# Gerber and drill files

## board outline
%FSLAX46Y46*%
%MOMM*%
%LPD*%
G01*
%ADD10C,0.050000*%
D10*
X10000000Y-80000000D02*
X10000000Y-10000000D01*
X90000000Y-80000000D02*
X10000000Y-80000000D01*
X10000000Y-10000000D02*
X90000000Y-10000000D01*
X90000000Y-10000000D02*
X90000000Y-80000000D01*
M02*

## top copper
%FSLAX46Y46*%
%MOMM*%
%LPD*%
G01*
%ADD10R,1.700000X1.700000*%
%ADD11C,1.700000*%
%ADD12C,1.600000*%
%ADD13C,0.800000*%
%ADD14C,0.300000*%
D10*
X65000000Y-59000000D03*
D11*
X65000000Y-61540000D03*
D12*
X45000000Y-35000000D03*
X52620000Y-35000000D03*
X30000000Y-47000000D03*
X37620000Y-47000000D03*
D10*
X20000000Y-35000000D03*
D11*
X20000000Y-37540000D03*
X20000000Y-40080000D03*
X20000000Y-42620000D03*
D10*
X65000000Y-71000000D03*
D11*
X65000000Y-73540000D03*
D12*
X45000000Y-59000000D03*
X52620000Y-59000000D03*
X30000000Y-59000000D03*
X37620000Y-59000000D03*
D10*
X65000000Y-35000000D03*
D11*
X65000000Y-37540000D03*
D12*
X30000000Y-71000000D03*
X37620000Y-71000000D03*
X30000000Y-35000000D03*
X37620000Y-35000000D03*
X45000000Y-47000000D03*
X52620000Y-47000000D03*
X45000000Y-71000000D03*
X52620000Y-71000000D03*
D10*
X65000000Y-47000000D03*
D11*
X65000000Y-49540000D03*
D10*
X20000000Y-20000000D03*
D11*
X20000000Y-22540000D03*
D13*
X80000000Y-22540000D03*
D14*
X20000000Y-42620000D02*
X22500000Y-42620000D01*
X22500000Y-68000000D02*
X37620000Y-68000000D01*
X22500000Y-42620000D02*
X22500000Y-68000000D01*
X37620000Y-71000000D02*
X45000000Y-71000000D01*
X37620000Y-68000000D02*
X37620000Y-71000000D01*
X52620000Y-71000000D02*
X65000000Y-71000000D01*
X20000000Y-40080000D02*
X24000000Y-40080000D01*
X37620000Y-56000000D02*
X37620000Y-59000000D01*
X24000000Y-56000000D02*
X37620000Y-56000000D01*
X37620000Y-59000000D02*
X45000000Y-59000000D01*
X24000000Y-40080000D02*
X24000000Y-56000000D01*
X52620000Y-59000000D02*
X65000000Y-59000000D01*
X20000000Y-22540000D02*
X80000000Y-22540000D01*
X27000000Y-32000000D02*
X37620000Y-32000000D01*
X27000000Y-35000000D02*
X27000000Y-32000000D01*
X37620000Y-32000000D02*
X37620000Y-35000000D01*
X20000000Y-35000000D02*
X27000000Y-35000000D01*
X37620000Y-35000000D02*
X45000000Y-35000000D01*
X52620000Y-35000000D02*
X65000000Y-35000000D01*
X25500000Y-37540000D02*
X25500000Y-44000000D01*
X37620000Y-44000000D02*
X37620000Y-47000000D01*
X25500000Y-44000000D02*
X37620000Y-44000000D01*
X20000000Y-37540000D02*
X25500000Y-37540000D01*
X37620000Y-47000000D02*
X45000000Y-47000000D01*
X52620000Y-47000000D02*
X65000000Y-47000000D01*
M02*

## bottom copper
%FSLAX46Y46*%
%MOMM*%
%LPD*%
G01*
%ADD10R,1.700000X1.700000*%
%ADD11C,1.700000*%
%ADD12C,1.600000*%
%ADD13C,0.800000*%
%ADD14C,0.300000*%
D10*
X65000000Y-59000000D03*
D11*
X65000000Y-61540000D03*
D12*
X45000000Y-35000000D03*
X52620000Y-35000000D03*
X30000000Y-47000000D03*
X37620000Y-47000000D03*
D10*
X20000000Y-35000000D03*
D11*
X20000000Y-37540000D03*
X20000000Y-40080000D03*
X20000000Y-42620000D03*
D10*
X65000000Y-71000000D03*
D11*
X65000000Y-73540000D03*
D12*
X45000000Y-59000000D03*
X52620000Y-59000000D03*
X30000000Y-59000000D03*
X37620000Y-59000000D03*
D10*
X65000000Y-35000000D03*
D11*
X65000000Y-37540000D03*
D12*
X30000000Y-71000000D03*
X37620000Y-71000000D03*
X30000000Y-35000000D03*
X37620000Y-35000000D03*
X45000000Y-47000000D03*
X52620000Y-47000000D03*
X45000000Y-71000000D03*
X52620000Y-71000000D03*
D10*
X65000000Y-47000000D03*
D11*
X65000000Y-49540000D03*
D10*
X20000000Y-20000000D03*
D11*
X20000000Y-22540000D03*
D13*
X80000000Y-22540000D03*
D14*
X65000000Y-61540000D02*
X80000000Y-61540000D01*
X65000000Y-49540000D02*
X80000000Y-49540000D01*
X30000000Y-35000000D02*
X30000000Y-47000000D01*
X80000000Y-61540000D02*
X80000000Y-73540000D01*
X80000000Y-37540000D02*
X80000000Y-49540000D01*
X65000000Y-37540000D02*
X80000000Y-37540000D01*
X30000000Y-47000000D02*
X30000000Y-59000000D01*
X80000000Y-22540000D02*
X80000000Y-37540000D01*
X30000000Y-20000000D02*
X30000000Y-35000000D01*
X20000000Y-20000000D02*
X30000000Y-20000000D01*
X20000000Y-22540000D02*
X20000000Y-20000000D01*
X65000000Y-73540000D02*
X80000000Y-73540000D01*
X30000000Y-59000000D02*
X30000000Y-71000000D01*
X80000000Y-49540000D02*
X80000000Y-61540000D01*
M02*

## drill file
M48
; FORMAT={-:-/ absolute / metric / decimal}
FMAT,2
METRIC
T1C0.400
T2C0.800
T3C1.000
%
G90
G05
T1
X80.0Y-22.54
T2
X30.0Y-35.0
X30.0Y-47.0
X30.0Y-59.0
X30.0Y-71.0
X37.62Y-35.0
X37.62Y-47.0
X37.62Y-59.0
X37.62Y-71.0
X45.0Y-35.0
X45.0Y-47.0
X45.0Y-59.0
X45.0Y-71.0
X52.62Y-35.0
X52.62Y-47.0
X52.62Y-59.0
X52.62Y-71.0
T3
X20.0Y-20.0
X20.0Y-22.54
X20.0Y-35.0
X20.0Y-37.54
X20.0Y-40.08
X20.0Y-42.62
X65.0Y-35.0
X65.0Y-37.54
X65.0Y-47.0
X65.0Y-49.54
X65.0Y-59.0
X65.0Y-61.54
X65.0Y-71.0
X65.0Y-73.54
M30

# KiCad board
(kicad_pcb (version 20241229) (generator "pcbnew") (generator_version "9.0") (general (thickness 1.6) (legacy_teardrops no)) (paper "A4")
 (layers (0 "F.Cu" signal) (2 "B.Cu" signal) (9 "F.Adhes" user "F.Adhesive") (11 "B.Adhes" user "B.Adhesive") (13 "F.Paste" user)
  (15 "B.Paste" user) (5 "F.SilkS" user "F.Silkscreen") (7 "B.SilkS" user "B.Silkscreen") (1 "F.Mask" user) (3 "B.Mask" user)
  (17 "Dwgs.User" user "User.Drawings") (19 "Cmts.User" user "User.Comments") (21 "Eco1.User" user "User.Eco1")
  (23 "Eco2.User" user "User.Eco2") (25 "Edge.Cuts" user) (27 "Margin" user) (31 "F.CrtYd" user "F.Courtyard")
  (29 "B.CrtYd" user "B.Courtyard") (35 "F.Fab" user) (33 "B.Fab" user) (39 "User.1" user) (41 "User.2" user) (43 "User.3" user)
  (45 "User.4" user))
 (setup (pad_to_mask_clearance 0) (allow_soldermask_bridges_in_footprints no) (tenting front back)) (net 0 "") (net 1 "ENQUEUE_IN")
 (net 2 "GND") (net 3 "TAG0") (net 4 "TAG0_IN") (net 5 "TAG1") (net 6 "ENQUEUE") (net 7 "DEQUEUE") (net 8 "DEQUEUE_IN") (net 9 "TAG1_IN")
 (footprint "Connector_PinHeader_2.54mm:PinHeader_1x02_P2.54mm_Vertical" (layer "F.Cu") (at 65 59)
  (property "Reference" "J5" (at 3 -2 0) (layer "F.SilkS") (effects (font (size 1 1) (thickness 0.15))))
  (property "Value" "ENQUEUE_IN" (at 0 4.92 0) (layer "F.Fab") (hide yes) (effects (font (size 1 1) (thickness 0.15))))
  (pad "1" thru_hole rect (at 0 0) (size 1.7 1.7) (drill 1) (layers "*.Cu" "*.Mask") (remove_unused_layers no) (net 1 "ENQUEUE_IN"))
  (pad "2" thru_hole circle (at 0 2.54) (size 1.7 1.7) (drill 1) (layers "*.Cu" "*.Mask") (remove_unused_layers no) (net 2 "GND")))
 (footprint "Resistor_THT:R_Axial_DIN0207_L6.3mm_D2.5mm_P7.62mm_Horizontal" (layer "F.Cu") (at 45 35)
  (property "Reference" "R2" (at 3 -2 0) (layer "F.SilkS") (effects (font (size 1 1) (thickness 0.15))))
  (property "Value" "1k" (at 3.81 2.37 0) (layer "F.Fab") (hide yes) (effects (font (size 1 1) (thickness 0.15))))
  (pad "1" thru_hole circle (at 0 0) (size 1.6 1.6) (drill 0.8) (layers "*.Cu" "*.Mask") (remove_unused_layers no) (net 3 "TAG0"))
  (pad "2" thru_hole circle (at 7.62 0) (size 1.6 1.6) (drill 0.8) (layers "*.Cu" "*.Mask") (remove_unused_layers no) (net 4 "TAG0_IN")))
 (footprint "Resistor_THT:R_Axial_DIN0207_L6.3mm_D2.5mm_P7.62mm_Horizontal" (layer "F.Cu") (at 30 47)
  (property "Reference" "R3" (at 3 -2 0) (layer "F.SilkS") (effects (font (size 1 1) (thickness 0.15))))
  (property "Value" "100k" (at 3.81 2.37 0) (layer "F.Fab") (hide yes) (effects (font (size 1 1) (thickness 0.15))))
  (pad "1" thru_hole circle (at 0 0) (size 1.6 1.6) (drill 0.8) (layers "*.Cu" "*.Mask") (remove_unused_layers no) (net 2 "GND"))
  (pad "2" thru_hole circle (at 7.62 0) (size 1.6 1.6) (drill 0.8) (layers "*.Cu" "*.Mask") (remove_unused_layers no) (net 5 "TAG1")))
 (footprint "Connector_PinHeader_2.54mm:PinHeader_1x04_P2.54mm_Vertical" (layer "F.Cu") (at 20 35)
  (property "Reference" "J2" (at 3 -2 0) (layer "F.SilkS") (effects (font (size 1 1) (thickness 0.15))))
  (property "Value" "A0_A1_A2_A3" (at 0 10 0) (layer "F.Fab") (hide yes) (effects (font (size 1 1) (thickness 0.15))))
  (pad "1" thru_hole rect (at 0 0) (size 1.7 1.7) (drill 1) (layers "*.Cu" "*.Mask") (remove_unused_layers no) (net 3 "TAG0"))
  (pad "2" thru_hole circle (at 0 2.54) (size 1.7 1.7) (drill 1) (layers "*.Cu" "*.Mask") (remove_unused_layers no) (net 5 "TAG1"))
  (pad "3" thru_hole circle (at 0 5.08) (size 1.7 1.7) (drill 1) (layers "*.Cu" "*.Mask") (remove_unused_layers no) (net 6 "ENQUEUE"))
  (pad "4" thru_hole circle (at 0 7.62) (size 1.7 1.7) (drill 1) (layers "*.Cu" "*.Mask") (remove_unused_layers no) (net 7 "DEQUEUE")))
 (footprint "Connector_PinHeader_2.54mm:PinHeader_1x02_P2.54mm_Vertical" (layer "F.Cu") (at 65 71)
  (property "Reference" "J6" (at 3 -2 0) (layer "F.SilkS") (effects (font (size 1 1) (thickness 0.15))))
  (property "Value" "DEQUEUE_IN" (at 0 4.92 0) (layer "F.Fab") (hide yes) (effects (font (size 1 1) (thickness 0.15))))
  (pad "1" thru_hole rect (at 0 0) (size 1.7 1.7) (drill 1) (layers "*.Cu" "*.Mask") (remove_unused_layers no) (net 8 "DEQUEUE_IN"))
  (pad "2" thru_hole circle (at 0 2.54) (size 1.7 1.7) (drill 1) (layers "*.Cu" "*.Mask") (remove_unused_layers no) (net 2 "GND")))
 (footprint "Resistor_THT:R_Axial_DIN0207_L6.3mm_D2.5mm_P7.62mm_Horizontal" (layer "F.Cu") (at 45 59)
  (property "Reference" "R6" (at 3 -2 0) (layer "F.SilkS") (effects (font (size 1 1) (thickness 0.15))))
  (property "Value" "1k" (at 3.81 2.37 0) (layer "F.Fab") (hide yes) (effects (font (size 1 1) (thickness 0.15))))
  (pad "1" thru_hole circle (at 0 0) (size 1.6 1.6) (drill 0.8) (layers "*.Cu" "*.Mask") (remove_unused_layers no) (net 6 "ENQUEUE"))
  (pad "2" thru_hole circle (at 7.62 0) (size 1.6 1.6) (drill 0.8) (layers "*.Cu" "*.Mask") (remove_unused_layers no) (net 1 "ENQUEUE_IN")))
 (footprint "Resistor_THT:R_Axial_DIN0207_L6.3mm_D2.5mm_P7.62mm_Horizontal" (layer "F.Cu") (at 30 59)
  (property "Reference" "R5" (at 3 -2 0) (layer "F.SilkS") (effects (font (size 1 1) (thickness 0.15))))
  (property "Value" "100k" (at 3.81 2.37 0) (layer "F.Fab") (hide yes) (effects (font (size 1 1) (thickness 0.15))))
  (pad "1" thru_hole circle (at 0 0) (size 1.6 1.6) (drill 0.8) (layers "*.Cu" "*.Mask") (remove_unused_layers no) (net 2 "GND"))
  (pad "2" thru_hole circle (at 7.62 0) (size 1.6 1.6) (drill 0.8) (layers "*.Cu" "*.Mask") (remove_unused_layers no) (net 6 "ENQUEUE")))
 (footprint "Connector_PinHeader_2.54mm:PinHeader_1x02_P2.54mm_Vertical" (layer "F.Cu") (at 65 35)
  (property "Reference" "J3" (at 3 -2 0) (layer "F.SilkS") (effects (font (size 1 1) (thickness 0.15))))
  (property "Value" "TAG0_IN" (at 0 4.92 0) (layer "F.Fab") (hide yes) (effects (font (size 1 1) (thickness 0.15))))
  (pad "1" thru_hole rect (at 0 0) (size 1.7 1.7) (drill 1) (layers "*.Cu" "*.Mask") (remove_unused_layers no) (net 4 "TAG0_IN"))
  (pad "2" thru_hole circle (at 0 2.54) (size 1.7 1.7) (drill 1) (layers "*.Cu" "*.Mask") (remove_unused_layers no) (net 2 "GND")))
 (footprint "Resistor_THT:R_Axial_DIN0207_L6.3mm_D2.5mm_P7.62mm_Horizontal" (layer "F.Cu") (at 30 71)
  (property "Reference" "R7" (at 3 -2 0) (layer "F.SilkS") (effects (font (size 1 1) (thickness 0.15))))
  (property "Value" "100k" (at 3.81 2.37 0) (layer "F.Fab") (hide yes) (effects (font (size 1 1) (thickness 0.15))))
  (pad "1" thru_hole circle (at 0 0) (size 1.6 1.6) (drill 0.8) (layers "*.Cu" "*.Mask") (remove_unused_layers no) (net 2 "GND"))
  (pad "2" thru_hole circle (at 7.62 0) (size 1.6 1.6) (drill 0.8) (layers "*.Cu" "*.Mask") (remove_unused_layers no) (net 7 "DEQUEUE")))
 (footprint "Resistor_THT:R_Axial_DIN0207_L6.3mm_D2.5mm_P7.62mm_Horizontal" (layer "F.Cu") (at 30 35)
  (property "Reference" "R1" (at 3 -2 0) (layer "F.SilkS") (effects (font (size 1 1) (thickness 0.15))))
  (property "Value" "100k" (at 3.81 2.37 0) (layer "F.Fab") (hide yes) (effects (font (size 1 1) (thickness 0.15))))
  (pad "1" thru_hole circle (at 0 0) (size 1.6 1.6) (drill 0.8) (layers "*.Cu" "*.Mask") (remove_unused_layers no) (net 2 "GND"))
  (pad "2" thru_hole circle (at 7.62 0) (size 1.6 1.6) (drill 0.8) (layers "*.Cu" "*.Mask") (remove_unused_layers no) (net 3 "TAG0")))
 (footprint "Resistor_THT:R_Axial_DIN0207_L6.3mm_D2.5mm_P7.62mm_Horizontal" (layer "F.Cu") (at 45 47)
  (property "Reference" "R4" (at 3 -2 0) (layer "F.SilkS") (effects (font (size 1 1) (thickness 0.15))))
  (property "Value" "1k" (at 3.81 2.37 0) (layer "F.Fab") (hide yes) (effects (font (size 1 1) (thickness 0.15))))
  (pad "1" thru_hole circle (at 0 0) (size 1.6 1.6) (drill 0.8) (layers "*.Cu" "*.Mask") (remove_unused_layers no) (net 5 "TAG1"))
  (pad "2" thru_hole circle (at 7.62 0) (size 1.6 1.6) (drill 0.8) (layers "*.Cu" "*.Mask") (remove_unused_layers no) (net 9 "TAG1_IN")))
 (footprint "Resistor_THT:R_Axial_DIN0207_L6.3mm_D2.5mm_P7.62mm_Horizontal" (layer "F.Cu") (at 45 71)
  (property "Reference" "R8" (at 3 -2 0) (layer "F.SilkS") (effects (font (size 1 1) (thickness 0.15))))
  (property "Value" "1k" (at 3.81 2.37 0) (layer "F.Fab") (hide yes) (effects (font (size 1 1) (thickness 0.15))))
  (pad "1" thru_hole circle (at 0 0) (size 1.6 1.6) (drill 0.8) (layers "*.Cu" "*.Mask") (remove_unused_layers no) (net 7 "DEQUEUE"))
  (pad "2" thru_hole circle (at 7.62 0) (size 1.6 1.6) (drill 0.8) (layers "*.Cu" "*.Mask") (remove_unused_layers no) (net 8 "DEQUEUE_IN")))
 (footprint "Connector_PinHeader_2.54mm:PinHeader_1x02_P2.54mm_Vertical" (layer "F.Cu") (at 65 47)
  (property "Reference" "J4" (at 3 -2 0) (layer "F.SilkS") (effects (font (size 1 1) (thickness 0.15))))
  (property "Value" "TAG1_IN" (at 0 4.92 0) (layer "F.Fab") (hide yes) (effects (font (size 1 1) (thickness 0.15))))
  (pad "1" thru_hole rect (at 0 0) (size 1.7 1.7) (drill 1) (layers "*.Cu" "*.Mask") (remove_unused_layers no) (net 9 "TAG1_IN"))
  (pad "2" thru_hole circle (at 0 2.54) (size 1.7 1.7) (drill 1) (layers "*.Cu" "*.Mask") (remove_unused_layers no) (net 2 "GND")))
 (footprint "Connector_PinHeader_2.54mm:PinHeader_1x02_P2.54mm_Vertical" (layer "F.Cu") (at 20 20)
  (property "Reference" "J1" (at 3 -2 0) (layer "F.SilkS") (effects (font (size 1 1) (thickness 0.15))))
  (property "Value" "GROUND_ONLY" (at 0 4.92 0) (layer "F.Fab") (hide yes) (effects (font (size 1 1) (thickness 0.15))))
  (pad "1" thru_hole rect (at 0 0) (size 1.7 1.7) (drill 1) (layers "*.Cu" "*.Mask") (remove_unused_layers no) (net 2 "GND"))
  (pad "2" thru_hole circle (at 0 2.54) (size 1.7 1.7) (drill 1) (layers "*.Cu" "*.Mask") (remove_unused_layers no) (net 2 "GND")))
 (gr_line (start 10 80) (end 10 10) (stroke (width 0.05) (type default)) (layer "Edge.Cuts"))
 (gr_line (start 90 80) (end 10 80) (stroke (width 0.05) (type default)) (layer "Edge.Cuts"))
 (gr_line (start 10 10) (end 90 10) (stroke (width 0.05) (type default)) (layer "Edge.Cuts"))
 (gr_line (start 90 10) (end 90 80) (stroke (width 0.05) (type default)) (layer "Edge.Cuts"))
 (segment (start 20 42.62) (end 22.5 42.62) (width 0.3) (layer "F.Cu") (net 7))
 (segment (start 22.5 68) (end 37.62 68) (width 0.3) (layer "F.Cu") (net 7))
 (segment (start 22.5 42.62) (end 22.5 68) (width 0.3) (layer "F.Cu") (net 7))
 (segment (start 37.62 71) (end 45 71) (width 0.3) (layer "F.Cu") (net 7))
 (segment (start 37.62 68) (end 37.62 71) (width 0.3) (layer "F.Cu") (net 7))
 (segment (start 52.62 71) (end 65 71) (width 0.3) (layer "F.Cu") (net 8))
 (segment (start 20 40.08) (end 24 40.08) (width 0.3) (layer "F.Cu") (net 6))
 (segment (start 37.62 56) (end 37.62 59) (width 0.3) (layer "F.Cu") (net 6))
 (segment (start 24 56) (end 37.62 56) (width 0.3) (layer "F.Cu") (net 6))
 (segment (start 37.62 59) (end 45 59) (width 0.3) (layer "F.Cu") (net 6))
 (segment (start 24 40.08) (end 24 56) (width 0.3) (layer "F.Cu") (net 6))
 (segment (start 52.62 59) (end 65 59) (width 0.3) (layer "F.Cu") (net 1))
 (segment (start 20 22.54) (end 80 22.54) (width 0.3) (layer "F.Cu") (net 2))
 (via (at 80 22.54) (size 0.8) (drill 0.4) (layers "F.Cu" "B.Cu") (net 2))
 (segment (start 65 61.54) (end 80 61.54) (width 0.3) (layer "B.Cu") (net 2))
 (segment (start 65 49.54) (end 80 49.54) (width 0.3) (layer "B.Cu") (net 2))
 (segment (start 30 35) (end 30 47) (width 0.3) (layer "B.Cu") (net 2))
 (segment (start 80 61.54) (end 80 73.54) (width 0.3) (layer "B.Cu") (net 2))
 (segment (start 80 37.54) (end 80 49.54) (width 0.3) (layer "B.Cu") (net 2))
 (segment (start 65 37.54) (end 80 37.54) (width 0.3) (layer "B.Cu") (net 2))
 (segment (start 30 47) (end 30 59) (width 0.3) (layer "B.Cu") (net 2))
 (segment (start 80 22.54) (end 80 37.54) (width 0.3) (layer "B.Cu") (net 2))
 (segment (start 30 20) (end 30 35) (width 0.3) (layer "B.Cu") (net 2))
 (segment (start 20 20) (end 30 20) (width 0.3) (layer "B.Cu") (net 2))
 (segment (start 20 22.54) (end 20 20) (width 0.3) (layer "B.Cu") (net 2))
 (segment (start 65 73.54) (end 80 73.54) (width 0.3) (layer "B.Cu") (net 2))
 (segment (start 30 59) (end 30 71) (width 0.3) (layer "B.Cu") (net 2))
 (segment (start 80 49.54) (end 80 61.54) (width 0.3) (layer "B.Cu") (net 2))
 (segment (start 27 32) (end 37.62 32) (width 0.3) (layer "F.Cu") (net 3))
 (segment (start 27 35) (end 27 32) (width 0.3) (layer "F.Cu") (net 3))
 (segment (start 37.62 32) (end 37.62 35) (width 0.3) (layer "F.Cu") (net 3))
 (segment (start 20 35) (end 27 35) (width 0.3) (layer "F.Cu") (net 3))
 (segment (start 37.62 35) (end 45 35) (width 0.3) (layer "F.Cu") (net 3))
 (segment (start 52.62 35) (end 65 35) (width 0.3) (layer "F.Cu") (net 4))
 (segment (start 25.5 37.54) (end 25.5 44) (width 0.3) (layer "F.Cu") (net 5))
 (segment (start 37.62 44) (end 37.62 47) (width 0.3) (layer "F.Cu") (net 5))
 (segment (start 25.5 44) (end 37.62 44) (width 0.3) (layer "F.Cu") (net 5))
 (segment (start 20 37.54) (end 25.5 37.54) (width 0.3) (layer "F.Cu") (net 5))
 (segment (start 37.62 47) (end 45 47) (width 0.3) (layer "F.Cu") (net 5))
 (segment (start 52.62 47) (end 65 47) (width 0.3) (layer "F.Cu") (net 9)))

